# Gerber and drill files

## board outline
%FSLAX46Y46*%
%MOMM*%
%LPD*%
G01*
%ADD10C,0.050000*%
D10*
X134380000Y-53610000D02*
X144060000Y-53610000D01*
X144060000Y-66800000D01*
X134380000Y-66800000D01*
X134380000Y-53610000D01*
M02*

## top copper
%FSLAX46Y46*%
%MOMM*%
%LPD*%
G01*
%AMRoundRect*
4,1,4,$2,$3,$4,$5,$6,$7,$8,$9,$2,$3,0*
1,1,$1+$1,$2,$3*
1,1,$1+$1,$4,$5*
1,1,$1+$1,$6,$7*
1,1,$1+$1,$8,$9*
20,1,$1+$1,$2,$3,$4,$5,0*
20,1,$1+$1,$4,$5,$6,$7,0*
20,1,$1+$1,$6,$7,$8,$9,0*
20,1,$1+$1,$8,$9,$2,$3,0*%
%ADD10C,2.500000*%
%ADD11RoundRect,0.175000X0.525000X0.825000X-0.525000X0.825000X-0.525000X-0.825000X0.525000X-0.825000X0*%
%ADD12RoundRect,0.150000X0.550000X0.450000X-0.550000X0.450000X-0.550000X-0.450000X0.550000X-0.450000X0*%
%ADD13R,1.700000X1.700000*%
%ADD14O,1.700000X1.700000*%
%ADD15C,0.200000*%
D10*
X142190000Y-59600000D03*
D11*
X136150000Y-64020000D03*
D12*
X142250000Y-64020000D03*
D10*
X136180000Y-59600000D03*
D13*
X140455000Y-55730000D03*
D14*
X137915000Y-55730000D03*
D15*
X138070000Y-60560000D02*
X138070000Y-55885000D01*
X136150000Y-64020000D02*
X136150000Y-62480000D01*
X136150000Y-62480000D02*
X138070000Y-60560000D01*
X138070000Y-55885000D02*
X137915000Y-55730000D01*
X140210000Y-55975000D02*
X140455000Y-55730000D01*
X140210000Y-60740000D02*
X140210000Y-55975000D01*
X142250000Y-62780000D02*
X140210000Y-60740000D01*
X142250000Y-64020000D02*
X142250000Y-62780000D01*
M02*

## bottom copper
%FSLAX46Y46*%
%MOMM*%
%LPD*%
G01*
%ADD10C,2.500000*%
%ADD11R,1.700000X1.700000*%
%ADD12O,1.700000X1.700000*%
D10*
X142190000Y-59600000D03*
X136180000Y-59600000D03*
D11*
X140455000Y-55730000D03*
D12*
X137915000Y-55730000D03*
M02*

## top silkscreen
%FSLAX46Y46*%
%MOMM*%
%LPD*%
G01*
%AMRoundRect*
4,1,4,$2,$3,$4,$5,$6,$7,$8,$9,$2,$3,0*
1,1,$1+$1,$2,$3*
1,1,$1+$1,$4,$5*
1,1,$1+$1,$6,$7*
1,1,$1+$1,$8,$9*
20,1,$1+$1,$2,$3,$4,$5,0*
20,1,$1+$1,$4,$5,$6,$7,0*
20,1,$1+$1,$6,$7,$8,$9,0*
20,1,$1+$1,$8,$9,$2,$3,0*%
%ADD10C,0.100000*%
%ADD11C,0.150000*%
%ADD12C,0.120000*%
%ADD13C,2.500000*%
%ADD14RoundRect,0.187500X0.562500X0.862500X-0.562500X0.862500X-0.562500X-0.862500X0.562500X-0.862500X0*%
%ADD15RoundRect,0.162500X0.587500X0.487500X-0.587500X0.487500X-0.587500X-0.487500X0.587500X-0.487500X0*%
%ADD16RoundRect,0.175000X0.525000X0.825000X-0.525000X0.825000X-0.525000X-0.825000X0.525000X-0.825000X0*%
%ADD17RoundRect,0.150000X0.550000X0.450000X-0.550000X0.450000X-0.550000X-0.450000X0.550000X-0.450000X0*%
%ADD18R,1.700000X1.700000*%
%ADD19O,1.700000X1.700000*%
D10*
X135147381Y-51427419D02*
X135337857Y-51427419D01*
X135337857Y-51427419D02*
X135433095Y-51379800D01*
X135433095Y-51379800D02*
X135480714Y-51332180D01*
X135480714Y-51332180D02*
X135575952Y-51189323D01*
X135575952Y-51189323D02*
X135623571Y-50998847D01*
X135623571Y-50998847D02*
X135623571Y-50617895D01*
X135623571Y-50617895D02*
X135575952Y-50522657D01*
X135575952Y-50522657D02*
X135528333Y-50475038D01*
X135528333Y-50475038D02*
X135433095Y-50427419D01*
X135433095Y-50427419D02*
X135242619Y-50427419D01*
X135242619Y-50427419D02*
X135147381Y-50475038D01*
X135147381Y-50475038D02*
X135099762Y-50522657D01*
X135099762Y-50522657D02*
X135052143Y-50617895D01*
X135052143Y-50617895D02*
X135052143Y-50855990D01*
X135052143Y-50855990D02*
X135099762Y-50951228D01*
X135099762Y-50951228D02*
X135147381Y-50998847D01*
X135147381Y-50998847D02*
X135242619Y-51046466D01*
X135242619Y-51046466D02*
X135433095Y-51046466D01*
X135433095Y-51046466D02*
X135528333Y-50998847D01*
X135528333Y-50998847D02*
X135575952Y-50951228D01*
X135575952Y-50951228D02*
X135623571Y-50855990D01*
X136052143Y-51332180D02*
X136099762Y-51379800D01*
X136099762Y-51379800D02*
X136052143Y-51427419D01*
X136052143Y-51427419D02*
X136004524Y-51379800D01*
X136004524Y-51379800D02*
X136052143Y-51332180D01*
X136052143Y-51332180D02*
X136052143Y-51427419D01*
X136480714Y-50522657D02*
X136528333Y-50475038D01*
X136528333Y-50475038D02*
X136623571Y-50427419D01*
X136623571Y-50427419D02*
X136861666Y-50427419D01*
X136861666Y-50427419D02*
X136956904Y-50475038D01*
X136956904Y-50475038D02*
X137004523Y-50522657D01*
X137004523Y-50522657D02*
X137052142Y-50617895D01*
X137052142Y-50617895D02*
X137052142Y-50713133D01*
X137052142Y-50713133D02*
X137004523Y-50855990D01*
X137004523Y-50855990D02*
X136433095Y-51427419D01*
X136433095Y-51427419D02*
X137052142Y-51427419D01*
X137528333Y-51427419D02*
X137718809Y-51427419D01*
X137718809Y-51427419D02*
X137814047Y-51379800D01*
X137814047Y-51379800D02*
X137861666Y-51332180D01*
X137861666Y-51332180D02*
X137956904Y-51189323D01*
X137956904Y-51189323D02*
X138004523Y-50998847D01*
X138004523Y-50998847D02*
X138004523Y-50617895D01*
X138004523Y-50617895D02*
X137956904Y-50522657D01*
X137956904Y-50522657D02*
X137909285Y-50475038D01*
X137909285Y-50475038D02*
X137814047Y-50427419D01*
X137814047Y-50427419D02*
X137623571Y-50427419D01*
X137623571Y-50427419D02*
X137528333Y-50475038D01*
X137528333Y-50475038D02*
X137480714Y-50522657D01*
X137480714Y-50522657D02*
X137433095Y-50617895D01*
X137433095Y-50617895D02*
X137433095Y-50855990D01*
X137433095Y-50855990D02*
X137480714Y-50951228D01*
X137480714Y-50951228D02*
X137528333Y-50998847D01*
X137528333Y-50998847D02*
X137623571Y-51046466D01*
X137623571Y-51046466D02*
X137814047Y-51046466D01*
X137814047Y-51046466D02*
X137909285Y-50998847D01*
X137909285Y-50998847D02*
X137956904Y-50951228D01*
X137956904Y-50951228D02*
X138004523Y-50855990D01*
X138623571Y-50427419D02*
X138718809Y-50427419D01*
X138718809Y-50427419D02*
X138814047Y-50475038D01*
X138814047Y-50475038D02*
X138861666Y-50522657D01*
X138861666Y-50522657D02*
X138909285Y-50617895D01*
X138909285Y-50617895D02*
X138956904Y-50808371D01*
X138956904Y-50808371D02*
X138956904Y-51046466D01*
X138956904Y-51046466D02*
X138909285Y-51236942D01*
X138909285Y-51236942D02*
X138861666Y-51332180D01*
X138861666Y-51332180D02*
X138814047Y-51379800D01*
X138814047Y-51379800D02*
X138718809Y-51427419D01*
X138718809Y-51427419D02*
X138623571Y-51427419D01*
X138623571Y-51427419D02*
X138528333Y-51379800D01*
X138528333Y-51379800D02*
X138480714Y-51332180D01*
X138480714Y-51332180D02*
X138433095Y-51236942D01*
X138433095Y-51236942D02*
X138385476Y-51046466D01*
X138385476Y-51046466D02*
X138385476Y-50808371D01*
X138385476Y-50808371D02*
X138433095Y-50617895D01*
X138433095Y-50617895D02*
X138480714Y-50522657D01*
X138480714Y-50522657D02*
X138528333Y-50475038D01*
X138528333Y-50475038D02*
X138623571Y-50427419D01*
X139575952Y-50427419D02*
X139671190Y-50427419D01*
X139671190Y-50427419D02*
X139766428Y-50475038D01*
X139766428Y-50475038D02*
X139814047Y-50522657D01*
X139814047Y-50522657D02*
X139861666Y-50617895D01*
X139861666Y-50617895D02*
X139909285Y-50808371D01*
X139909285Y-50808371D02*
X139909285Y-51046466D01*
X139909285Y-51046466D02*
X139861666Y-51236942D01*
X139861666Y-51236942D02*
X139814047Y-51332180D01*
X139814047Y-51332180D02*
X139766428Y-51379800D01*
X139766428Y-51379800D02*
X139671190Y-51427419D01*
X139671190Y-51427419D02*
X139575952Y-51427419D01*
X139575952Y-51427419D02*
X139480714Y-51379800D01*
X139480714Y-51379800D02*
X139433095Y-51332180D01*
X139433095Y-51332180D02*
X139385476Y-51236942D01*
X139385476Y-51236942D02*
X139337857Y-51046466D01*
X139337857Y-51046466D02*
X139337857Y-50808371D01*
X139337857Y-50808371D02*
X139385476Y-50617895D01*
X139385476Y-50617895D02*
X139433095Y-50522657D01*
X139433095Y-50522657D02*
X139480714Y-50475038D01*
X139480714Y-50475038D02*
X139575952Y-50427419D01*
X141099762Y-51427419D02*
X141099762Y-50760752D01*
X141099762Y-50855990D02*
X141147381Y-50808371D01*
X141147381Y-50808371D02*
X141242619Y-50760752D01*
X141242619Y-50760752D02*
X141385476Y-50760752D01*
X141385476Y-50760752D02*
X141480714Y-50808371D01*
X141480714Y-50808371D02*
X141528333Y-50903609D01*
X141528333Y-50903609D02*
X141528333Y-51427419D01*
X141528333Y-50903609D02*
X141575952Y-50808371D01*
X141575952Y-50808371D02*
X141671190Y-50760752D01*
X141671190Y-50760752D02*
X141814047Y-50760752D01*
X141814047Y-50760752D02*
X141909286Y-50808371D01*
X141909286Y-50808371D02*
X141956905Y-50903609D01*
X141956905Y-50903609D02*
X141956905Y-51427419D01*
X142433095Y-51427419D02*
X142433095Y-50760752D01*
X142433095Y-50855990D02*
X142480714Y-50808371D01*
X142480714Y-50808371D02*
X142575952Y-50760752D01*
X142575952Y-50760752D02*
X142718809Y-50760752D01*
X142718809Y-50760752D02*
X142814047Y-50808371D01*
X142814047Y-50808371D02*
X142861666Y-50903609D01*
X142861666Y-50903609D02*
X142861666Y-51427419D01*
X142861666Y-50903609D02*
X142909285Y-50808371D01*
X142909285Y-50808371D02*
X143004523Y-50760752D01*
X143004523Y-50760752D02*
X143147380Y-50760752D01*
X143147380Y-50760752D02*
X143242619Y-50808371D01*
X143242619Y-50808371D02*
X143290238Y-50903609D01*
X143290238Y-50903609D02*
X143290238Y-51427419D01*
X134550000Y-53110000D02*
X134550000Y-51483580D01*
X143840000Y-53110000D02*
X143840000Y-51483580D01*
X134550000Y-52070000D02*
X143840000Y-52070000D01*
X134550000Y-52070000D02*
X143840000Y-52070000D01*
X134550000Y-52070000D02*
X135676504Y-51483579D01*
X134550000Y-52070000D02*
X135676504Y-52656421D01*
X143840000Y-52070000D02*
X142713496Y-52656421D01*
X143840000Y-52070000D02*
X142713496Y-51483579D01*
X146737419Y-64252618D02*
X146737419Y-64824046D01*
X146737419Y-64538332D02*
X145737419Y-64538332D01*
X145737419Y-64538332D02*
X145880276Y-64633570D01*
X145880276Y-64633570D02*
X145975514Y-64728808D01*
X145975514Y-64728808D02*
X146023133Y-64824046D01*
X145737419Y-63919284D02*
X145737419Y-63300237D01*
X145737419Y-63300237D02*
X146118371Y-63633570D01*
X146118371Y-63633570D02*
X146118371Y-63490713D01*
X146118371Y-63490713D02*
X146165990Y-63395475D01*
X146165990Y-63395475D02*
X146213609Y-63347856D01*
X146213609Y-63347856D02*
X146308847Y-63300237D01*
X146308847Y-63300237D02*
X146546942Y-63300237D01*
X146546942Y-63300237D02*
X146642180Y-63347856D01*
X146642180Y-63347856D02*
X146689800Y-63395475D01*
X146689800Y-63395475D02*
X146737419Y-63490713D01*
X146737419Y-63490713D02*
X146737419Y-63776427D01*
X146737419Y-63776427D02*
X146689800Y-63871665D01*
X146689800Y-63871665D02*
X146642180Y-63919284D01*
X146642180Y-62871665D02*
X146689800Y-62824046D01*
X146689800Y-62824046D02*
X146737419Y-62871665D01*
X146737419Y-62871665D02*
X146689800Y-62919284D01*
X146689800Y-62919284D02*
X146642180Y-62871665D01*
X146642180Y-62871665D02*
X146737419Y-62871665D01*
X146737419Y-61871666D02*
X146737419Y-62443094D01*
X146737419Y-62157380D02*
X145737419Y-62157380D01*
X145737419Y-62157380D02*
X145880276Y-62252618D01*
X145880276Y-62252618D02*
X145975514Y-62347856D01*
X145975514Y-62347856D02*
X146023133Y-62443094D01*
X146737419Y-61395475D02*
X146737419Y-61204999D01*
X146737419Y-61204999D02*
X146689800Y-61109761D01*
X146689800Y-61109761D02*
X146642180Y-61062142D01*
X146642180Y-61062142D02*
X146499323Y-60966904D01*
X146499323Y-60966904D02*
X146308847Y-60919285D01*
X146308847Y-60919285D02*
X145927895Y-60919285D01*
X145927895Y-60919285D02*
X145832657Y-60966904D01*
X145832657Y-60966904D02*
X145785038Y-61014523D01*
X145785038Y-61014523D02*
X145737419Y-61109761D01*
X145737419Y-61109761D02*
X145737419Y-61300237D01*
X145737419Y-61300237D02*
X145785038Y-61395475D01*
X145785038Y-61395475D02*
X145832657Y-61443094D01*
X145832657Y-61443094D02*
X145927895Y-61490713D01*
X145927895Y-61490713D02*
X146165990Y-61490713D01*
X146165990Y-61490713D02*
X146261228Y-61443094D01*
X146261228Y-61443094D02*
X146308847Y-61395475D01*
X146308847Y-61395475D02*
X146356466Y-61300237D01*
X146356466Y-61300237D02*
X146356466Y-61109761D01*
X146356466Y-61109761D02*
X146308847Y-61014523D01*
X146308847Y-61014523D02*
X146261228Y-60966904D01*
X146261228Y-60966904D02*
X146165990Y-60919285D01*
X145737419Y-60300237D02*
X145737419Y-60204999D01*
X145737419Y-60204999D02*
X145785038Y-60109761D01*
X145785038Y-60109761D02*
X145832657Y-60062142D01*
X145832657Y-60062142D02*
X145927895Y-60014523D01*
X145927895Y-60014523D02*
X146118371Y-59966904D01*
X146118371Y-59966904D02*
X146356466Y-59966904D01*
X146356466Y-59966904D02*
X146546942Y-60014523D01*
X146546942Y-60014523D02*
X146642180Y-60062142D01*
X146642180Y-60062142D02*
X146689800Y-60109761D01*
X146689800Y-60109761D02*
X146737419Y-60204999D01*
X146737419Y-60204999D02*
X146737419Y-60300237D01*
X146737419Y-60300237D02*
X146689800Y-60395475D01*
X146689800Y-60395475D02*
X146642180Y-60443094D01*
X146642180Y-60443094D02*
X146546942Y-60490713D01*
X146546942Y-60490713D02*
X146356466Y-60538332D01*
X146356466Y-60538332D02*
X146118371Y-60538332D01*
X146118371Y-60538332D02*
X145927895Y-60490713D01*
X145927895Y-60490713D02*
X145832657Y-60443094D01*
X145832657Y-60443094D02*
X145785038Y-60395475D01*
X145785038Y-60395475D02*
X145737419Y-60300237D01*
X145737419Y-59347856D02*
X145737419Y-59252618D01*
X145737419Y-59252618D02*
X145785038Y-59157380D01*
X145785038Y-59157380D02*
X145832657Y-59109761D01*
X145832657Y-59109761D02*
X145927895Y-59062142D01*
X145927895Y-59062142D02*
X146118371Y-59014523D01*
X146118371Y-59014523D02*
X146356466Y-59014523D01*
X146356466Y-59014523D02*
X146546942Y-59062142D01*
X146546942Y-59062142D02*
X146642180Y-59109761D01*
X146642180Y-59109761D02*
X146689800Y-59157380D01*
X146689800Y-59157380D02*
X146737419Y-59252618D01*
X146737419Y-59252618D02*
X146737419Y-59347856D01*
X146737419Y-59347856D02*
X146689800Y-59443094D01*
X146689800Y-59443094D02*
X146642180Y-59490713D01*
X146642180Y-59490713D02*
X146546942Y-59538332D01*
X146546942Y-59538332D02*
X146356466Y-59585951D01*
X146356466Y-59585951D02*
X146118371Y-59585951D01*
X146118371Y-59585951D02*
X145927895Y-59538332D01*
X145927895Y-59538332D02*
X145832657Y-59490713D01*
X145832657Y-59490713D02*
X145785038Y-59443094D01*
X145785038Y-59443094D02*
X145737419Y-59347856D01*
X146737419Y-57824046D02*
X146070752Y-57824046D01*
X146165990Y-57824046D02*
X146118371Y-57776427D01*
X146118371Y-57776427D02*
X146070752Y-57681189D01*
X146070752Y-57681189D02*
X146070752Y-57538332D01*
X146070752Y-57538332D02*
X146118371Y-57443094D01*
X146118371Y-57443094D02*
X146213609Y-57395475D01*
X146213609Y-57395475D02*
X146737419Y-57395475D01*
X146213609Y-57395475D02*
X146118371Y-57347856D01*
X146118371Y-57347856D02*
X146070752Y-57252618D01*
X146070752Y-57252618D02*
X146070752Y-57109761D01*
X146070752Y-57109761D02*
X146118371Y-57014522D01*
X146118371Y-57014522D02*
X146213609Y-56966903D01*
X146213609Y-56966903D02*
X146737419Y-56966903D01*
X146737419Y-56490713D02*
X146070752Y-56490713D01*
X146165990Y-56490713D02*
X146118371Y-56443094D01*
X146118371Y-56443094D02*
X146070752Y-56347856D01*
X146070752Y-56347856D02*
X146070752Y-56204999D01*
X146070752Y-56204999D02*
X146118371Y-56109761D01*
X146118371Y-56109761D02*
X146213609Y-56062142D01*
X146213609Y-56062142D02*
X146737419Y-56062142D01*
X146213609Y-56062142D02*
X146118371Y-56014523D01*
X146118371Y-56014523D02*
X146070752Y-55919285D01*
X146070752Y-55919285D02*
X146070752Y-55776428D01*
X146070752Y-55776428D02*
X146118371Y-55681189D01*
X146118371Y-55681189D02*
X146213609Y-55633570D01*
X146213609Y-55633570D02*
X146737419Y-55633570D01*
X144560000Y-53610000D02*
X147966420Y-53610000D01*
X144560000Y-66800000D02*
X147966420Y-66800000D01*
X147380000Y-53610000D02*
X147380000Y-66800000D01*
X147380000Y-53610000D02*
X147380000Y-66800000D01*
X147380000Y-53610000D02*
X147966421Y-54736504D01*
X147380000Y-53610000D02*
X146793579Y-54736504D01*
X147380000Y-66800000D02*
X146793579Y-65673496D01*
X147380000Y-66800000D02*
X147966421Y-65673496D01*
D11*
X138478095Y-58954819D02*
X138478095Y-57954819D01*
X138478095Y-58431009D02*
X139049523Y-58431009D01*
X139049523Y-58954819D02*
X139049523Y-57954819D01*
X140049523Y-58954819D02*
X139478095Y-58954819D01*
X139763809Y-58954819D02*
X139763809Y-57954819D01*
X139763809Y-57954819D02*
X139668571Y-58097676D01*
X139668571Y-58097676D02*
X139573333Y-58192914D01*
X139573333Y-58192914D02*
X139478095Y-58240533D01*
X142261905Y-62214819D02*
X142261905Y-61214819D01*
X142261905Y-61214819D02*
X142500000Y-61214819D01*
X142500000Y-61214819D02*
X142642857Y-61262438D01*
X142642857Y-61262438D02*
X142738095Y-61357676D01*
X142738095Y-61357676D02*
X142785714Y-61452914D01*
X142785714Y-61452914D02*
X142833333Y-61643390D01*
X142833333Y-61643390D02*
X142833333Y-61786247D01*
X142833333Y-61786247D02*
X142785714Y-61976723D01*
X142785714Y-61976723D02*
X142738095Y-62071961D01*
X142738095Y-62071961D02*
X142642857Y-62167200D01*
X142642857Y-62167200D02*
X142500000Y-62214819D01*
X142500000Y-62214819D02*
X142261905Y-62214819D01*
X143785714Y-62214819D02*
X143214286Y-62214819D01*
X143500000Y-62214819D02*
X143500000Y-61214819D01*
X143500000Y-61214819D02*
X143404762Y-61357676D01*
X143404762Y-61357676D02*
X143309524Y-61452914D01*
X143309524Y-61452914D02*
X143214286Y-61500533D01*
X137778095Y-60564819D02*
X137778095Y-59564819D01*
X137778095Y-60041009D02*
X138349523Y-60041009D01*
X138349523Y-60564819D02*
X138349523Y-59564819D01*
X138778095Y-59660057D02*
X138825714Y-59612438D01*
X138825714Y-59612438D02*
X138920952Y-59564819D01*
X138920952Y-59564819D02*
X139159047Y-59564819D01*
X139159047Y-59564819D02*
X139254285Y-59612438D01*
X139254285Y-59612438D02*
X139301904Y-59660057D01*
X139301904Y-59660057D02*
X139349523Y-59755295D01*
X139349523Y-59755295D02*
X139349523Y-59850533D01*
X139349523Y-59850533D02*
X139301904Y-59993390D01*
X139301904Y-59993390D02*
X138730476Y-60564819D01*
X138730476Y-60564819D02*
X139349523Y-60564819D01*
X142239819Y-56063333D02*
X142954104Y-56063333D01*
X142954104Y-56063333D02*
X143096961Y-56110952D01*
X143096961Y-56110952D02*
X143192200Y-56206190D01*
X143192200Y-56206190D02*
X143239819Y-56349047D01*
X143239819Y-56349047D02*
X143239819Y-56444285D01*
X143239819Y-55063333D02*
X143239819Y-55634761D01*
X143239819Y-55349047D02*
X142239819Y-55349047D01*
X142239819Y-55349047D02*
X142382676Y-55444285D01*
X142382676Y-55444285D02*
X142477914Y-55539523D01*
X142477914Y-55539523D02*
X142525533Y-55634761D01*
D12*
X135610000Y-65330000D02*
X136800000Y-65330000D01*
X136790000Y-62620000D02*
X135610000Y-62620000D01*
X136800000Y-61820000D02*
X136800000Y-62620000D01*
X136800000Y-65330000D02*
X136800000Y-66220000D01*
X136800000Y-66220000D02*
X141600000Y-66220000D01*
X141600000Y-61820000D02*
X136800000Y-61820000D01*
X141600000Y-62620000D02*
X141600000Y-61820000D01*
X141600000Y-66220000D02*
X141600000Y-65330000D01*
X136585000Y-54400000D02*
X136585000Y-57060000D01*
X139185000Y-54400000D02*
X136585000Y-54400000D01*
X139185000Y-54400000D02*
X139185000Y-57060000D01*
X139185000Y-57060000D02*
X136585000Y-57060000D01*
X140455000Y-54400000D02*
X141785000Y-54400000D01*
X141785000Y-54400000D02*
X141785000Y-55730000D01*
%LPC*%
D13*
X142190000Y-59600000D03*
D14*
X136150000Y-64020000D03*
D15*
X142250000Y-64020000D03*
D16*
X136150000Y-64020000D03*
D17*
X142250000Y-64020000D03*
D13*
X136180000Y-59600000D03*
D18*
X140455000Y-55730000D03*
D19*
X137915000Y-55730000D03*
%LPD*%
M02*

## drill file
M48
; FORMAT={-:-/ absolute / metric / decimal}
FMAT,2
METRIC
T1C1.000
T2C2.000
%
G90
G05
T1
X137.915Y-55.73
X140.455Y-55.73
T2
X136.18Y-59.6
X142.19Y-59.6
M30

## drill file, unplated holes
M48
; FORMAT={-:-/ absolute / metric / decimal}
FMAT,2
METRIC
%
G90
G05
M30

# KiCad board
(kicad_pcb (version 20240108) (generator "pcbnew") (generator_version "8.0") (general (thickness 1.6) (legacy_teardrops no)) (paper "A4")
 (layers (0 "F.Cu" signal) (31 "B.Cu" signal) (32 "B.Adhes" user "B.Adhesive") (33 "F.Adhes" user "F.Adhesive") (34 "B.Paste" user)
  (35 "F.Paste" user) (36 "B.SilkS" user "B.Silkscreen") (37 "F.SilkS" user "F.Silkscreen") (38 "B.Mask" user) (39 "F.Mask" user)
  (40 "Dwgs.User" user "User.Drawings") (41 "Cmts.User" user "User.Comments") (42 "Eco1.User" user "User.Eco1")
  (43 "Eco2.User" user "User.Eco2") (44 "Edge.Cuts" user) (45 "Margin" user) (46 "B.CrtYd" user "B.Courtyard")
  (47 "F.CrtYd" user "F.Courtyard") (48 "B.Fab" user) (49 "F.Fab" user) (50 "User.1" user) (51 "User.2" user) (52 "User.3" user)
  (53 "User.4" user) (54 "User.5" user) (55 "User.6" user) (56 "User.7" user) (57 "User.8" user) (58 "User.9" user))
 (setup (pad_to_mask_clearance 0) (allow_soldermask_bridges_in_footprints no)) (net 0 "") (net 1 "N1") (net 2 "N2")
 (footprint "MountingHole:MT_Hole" (layer "F.Cu") (at 142.19 59.6)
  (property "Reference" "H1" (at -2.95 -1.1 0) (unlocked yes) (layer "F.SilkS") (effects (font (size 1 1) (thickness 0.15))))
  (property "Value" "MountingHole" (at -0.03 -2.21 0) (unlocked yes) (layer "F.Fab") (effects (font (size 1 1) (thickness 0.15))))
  (pad "1" thru_hole circle (at 0 0) (size 2.5 2.5) (drill 2) (layers "*.Cu" "*.Mask") (remove_unused_layers no)))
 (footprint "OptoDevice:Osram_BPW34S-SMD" (layer "F.Cu") (at 139.2 64.02)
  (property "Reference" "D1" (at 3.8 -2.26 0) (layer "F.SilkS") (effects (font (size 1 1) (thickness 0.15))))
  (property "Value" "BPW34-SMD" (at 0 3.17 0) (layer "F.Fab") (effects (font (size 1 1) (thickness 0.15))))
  (fp_line (start -3.59 1.31) (end -2.4 1.31) (stroke (width 0.12) (type solid)) (layer "F.SilkS"))
  (fp_line (start -2.41 -1.4) (end -3.59 -1.4) (stroke (width 0.12) (type solid)) (layer "F.SilkS"))
  (fp_line (start -2.4 -2.2) (end -2.4 -1.4) (stroke (width 0.12) (type solid)) (layer "F.SilkS"))
  (fp_line (start -2.4 1.31) (end -2.4 2.2) (stroke (width 0.12) (type solid)) (layer "F.SilkS"))
  (fp_line (start -2.4 2.2) (end 2.4 2.2) (stroke (width 0.12) (type solid)) (layer "F.SilkS"))
  (fp_line (start 2.4 -2.2) (end -2.4 -2.2) (stroke (width 0.12) (type solid)) (layer "F.SilkS"))
  (fp_line (start 2.4 -1.4) (end 2.4 -2.2) (stroke (width 0.12) (type solid)) (layer "F.SilkS"))
  (fp_line (start 2.4 2.2) (end 2.4 1.31) (stroke (width 0.12) (type solid)) (layer "F.SilkS"))
  (pad "" smd roundrect (at -3.05 0 180) (size 1.3 1.9) (layers "F.Paste") (roundrect_rratio 0.125))
  (pad "" smd roundrect (at -3.05 0 180) (size 1.5 2.1) (layers "F.Mask") (roundrect_rratio 0.125))
  (pad "" smd roundrect (at 3.05 0 180) (size 1.3 1.1) (layers "F.Paste") (roundrect_rratio 0.125))
  (pad "" smd roundrect (at 3.05 0 180) (size 1.5 1.3) (layers "F.Mask") (roundrect_rratio 0.125))
  (pad "1" smd roundrect (at -3.05 0 180) (size 1.4 2) (layers "F.Cu" "F.Mask") (roundrect_rratio 0.125) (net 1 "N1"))
  (pad "2" smd roundrect (at 3.05 0 180) (size 1.4 1.2) (layers "F.Cu" "F.Mask") (roundrect_rratio 0.125) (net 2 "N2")))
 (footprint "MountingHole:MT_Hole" (layer "F.Cu") (at 136.18 59.6)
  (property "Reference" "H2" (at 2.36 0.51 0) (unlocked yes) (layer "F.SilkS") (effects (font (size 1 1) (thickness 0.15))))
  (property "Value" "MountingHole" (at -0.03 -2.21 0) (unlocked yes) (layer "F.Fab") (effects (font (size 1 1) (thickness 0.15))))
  (pad "1" thru_hole circle (at 0 0) (size 2.5 2.5) (drill 2) (layers "*.Cu" "*.Mask") (remove_unused_layers no)))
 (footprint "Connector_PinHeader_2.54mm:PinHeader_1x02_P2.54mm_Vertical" (layer "F.Cu") (at 140.455 55.73 -90)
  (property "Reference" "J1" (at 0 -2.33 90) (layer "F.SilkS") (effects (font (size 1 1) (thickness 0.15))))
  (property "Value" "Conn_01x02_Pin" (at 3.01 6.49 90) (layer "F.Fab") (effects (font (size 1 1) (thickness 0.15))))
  (fp_line (start -1.33 3.87) (end 1.33 3.87) (stroke (width 0.12) (type solid)) (layer "F.SilkS"))
  (fp_line (start -1.33 1.27) (end -1.33 3.87) (stroke (width 0.12) (type solid)) (layer "F.SilkS"))
  (fp_line (start -1.33 1.27) (end 1.33 1.27) (stroke (width 0.12) (type solid)) (layer "F.SilkS"))
  (fp_line (start 1.33 1.27) (end 1.33 3.87) (stroke (width 0.12) (type solid)) (layer "F.SilkS"))
  (fp_line (start -1.33 0) (end -1.33 -1.33) (stroke (width 0.12) (type solid)) (layer "F.SilkS"))
  (fp_line (start -1.33 -1.33) (end 0 -1.33) (stroke (width 0.12) (type solid)) (layer "F.SilkS"))
  (pad "1" thru_hole rect (at 0 0 270) (size 1.7 1.7) (drill 1) (layers "*.Cu" "*.Mask") (remove_unused_layers no) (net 2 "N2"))
  (pad "2" thru_hole oval (at 0 2.54 270) (size 1.7 1.7) (drill 1) (layers "*.Cu" "*.Mask") (remove_unused_layers no) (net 1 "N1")))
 (gr_rect (start 134.38 53.61) (end 144.06 66.8) (stroke (width 0.05) (type default)) (fill none) (layer "Edge.Cuts"))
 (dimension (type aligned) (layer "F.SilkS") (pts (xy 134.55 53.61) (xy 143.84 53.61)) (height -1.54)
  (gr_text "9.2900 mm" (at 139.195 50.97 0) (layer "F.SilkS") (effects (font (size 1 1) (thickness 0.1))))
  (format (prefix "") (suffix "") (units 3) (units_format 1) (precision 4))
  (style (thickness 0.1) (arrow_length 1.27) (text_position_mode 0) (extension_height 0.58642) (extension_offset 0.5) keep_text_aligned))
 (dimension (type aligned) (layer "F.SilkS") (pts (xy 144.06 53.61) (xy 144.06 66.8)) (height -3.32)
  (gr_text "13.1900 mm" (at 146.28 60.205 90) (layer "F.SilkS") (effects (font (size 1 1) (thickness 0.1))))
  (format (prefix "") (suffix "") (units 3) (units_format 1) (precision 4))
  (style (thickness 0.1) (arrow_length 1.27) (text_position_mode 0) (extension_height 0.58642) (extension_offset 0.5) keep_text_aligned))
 (segment (start 138.07 60.56) (end 138.07 55.885) (width 0.2) (layer "F.Cu") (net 1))
 (segment (start 136.15 64.02) (end 136.15 62.48) (width 0.2) (layer "F.Cu") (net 1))
 (segment (start 136.15 62.48) (end 138.07 60.56) (width 0.2) (layer "F.Cu") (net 1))
 (segment (start 138.07 55.885) (end 137.915 55.73) (width 0.2) (layer "F.Cu") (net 1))
 (segment (start 140.21 55.975) (end 140.455 55.73) (width 0.2) (layer "F.Cu") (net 2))
 (segment (start 140.21 60.74) (end 140.21 55.975) (width 0.2) (layer "F.Cu") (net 2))
 (segment (start 142.25 62.78) (end 140.21 60.74) (width 0.2) (layer "F.Cu") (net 2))
 (segment (start 142.25 64.02) (end 142.25 62.78) (width 0.2) (layer "F.Cu") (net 2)))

